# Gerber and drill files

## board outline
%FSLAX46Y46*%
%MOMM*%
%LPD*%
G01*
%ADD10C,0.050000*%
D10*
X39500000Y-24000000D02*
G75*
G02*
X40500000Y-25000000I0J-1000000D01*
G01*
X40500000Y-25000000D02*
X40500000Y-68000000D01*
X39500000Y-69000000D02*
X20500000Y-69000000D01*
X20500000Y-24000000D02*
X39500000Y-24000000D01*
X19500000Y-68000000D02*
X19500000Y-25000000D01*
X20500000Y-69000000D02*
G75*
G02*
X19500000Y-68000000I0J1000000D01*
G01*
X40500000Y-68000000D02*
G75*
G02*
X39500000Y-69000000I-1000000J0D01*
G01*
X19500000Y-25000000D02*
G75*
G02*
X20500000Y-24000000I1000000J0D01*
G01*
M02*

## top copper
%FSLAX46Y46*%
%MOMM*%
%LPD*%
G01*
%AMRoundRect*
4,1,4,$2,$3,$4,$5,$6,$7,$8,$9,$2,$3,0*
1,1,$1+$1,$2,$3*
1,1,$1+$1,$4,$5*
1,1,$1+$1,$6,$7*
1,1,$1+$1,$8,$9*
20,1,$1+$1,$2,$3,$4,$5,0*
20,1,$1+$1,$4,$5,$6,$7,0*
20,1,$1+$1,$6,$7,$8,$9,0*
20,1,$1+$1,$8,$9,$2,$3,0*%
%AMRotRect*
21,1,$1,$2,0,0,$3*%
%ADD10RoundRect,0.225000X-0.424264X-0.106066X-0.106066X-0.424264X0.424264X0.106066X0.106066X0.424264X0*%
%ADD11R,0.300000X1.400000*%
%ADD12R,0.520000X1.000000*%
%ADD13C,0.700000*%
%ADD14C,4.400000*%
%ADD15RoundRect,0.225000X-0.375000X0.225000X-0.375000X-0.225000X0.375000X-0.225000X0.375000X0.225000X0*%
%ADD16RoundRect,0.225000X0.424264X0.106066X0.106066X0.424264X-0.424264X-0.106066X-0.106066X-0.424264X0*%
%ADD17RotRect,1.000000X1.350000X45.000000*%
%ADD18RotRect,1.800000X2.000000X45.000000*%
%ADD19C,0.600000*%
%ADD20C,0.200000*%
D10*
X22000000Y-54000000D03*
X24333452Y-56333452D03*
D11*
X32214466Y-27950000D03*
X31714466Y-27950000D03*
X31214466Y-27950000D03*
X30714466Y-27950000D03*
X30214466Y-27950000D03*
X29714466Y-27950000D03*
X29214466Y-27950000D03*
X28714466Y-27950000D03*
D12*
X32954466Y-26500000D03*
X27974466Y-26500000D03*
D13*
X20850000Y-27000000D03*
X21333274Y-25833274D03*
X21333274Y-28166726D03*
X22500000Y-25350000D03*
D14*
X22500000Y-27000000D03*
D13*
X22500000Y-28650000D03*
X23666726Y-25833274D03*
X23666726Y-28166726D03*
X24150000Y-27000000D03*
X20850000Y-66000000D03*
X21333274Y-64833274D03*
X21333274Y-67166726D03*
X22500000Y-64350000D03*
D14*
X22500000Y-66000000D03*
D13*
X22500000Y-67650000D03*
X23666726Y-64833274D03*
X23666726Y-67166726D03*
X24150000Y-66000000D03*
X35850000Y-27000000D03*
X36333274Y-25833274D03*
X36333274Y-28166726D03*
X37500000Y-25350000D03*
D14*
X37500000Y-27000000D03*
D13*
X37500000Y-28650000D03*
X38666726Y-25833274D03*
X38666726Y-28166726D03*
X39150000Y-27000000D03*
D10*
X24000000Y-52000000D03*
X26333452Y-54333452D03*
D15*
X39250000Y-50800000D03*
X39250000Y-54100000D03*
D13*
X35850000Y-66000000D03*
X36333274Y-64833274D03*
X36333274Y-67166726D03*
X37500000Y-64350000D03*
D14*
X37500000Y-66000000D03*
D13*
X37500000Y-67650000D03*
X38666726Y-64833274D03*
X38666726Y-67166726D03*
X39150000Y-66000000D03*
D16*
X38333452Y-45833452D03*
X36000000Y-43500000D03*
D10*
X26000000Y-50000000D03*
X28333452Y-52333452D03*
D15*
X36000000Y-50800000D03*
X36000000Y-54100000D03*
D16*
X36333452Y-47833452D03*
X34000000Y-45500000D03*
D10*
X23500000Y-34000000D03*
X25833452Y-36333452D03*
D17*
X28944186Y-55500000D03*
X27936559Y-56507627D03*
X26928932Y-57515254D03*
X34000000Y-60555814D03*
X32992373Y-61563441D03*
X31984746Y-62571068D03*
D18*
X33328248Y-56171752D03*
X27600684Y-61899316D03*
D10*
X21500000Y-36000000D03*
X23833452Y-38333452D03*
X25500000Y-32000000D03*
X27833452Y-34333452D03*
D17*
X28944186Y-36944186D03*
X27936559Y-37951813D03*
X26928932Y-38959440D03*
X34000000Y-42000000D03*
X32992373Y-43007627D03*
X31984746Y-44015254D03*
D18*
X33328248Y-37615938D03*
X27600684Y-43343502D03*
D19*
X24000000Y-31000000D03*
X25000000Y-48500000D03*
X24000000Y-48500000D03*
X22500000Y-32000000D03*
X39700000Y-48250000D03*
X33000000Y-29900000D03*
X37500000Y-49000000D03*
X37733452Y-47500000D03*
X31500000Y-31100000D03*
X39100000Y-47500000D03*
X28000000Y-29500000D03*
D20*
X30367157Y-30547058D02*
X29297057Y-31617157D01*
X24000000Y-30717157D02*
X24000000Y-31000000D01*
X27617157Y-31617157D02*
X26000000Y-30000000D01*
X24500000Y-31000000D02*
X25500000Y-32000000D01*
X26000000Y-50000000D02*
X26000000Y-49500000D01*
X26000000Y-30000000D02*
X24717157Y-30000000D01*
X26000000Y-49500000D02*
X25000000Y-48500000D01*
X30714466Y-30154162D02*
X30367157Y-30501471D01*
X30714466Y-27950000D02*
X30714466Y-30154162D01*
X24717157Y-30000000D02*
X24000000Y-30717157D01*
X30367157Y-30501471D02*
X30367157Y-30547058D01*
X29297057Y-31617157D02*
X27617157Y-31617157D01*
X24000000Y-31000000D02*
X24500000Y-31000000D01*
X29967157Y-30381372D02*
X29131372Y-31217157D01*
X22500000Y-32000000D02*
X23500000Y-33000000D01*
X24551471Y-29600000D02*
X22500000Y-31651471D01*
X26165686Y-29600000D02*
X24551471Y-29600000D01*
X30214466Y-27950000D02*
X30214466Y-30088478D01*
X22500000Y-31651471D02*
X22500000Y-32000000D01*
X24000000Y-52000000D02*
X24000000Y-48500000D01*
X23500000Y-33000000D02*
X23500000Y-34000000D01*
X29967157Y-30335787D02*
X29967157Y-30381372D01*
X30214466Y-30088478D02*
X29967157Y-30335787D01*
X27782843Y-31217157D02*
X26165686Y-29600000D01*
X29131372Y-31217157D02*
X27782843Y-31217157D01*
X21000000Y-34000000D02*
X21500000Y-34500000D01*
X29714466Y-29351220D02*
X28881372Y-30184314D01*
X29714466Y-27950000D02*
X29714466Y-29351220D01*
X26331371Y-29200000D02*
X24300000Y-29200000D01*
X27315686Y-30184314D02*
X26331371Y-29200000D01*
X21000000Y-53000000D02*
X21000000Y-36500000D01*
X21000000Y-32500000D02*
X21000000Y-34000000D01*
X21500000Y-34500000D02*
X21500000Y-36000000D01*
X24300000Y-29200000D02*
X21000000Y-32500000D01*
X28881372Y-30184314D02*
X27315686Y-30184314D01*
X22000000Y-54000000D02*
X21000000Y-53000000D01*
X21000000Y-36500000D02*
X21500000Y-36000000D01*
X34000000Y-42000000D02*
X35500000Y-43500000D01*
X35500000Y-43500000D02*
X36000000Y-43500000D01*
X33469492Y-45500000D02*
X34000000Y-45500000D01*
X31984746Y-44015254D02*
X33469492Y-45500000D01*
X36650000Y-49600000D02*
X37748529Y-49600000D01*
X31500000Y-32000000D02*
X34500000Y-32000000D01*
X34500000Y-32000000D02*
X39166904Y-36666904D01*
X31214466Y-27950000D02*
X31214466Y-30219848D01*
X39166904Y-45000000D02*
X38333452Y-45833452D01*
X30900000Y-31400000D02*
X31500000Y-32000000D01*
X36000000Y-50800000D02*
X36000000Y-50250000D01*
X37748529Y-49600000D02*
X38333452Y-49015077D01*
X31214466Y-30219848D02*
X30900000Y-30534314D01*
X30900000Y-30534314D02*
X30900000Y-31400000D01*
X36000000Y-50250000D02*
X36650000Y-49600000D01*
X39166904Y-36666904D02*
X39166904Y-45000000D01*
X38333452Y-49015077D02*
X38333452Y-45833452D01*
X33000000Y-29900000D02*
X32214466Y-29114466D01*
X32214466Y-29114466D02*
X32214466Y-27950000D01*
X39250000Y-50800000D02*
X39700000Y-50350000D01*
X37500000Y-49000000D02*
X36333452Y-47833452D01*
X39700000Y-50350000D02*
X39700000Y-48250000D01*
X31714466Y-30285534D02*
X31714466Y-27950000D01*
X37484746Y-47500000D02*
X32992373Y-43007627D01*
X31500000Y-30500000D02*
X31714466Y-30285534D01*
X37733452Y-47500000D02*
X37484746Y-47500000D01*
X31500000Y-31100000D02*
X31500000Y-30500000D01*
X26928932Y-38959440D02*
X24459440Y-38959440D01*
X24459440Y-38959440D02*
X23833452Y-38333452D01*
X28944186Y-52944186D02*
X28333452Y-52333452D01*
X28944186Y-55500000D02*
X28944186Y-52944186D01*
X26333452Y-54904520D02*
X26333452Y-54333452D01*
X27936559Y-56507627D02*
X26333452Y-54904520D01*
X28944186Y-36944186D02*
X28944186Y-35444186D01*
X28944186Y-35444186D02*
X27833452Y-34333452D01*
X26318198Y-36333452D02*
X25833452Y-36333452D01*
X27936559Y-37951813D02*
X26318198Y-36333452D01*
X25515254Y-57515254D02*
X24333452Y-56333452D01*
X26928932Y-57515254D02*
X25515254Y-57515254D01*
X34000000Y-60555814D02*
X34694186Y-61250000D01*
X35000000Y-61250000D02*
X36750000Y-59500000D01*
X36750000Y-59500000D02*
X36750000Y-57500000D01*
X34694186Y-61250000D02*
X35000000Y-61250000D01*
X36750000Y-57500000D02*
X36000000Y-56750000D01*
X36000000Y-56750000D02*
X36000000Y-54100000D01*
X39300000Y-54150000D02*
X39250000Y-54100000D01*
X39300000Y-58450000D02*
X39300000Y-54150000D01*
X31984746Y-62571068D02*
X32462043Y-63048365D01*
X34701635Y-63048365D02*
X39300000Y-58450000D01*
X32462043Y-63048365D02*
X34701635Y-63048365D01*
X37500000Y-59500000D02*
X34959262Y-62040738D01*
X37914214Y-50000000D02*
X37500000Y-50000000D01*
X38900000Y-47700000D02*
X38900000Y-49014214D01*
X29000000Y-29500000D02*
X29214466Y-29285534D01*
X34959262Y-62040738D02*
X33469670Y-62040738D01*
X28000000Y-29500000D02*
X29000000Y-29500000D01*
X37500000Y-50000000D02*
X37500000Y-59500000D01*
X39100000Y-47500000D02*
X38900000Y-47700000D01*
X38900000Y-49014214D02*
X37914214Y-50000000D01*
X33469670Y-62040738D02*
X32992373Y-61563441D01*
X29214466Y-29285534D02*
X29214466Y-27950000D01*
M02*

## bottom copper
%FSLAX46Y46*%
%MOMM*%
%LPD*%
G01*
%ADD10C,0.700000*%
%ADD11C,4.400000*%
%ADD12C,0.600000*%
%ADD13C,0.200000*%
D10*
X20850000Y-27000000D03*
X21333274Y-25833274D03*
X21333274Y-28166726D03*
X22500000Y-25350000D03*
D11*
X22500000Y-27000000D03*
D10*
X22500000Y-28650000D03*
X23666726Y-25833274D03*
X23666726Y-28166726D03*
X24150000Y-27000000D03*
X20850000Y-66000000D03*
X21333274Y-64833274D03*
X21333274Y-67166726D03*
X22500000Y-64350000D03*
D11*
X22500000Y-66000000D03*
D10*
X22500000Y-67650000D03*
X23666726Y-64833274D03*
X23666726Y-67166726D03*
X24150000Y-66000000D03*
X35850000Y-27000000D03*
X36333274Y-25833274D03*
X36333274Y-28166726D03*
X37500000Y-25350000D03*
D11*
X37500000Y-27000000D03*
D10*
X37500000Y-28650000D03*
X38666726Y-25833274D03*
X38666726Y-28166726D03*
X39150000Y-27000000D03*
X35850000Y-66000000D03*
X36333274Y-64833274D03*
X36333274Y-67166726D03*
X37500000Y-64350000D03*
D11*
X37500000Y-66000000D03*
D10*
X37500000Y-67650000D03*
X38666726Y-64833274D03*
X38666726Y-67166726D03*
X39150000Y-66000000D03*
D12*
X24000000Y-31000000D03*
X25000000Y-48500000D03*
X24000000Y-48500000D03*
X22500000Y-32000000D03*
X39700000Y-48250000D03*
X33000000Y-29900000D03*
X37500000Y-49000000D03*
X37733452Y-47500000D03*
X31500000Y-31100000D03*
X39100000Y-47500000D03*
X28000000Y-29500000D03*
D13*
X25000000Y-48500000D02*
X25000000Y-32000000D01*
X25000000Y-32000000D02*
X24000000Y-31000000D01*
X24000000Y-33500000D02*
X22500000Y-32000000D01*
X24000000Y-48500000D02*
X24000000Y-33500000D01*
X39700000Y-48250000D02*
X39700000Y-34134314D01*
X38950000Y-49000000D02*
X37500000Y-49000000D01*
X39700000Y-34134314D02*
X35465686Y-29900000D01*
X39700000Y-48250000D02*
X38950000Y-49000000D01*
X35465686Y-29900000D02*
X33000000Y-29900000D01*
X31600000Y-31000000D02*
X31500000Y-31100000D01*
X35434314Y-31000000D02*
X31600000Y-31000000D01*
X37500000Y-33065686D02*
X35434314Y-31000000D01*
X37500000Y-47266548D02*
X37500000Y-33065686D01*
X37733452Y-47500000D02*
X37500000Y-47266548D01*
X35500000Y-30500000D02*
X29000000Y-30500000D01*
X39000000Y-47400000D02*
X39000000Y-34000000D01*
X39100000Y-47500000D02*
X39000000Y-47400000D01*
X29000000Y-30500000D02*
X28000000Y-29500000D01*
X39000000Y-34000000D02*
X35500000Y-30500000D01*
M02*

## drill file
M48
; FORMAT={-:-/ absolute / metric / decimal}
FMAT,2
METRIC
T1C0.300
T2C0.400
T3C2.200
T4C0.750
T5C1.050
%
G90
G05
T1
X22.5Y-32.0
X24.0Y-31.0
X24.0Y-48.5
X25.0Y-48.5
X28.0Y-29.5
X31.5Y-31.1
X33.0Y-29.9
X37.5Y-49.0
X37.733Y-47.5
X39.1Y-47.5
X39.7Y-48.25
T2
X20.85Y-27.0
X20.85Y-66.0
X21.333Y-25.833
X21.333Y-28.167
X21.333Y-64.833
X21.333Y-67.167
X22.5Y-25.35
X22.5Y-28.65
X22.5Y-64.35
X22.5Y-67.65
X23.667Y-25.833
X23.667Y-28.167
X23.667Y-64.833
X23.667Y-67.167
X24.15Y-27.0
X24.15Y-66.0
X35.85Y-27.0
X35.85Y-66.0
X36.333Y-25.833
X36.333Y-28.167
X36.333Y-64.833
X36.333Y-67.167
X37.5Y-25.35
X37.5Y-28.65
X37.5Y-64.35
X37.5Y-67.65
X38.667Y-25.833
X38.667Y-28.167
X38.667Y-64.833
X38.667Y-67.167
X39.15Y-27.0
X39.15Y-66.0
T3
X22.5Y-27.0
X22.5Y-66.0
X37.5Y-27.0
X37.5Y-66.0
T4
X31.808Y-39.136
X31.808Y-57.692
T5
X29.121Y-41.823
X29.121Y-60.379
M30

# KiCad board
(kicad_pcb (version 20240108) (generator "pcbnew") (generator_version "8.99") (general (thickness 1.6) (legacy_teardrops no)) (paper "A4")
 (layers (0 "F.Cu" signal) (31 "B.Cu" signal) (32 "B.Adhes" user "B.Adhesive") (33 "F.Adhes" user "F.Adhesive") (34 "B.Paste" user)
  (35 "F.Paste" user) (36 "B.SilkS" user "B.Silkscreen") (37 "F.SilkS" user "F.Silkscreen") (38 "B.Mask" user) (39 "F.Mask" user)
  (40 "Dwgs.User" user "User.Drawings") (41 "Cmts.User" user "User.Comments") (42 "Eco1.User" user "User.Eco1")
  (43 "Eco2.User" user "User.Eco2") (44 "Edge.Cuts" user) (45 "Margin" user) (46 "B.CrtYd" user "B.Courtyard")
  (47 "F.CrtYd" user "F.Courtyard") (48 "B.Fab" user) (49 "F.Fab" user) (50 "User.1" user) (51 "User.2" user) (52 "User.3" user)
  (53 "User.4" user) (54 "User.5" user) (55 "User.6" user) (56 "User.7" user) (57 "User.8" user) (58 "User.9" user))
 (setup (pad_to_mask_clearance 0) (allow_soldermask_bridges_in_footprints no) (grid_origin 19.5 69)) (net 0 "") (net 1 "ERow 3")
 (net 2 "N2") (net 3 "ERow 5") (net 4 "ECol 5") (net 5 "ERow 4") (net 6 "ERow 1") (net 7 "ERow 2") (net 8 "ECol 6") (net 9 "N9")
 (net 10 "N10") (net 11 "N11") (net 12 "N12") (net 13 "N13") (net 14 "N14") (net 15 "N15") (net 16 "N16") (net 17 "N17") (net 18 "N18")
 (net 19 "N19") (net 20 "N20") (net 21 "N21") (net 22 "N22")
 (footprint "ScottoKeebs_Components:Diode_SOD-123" (layer "F.Cu") (at 23.166726 55.166726 -45)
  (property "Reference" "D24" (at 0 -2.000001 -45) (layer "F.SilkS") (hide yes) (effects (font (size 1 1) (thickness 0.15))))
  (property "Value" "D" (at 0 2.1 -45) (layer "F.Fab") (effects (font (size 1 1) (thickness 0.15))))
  (pad "1" smd roundrect (at -1.65 0 315) (size 0.9 1.2) (layers "F.Cu" "F.Paste" "F.Mask") (roundrect_rratio 0.25) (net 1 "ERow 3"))
  (pad "2" smd roundrect (at 1.65 0 315) (size 0.9 1.2) (layers "F.Cu" "F.Paste" "F.Mask") (roundrect_rratio 0.25) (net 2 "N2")))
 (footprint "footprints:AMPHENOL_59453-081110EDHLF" (layer "F.Cu") (at 30.464466 26.1 180)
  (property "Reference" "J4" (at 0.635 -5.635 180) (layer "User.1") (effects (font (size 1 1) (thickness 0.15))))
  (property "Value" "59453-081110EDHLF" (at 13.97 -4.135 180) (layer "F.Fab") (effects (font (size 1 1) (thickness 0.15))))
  (pad "1" smd rect (at -1.75 -1.85 180) (size 0.3 1.4) (layers "F.Cu" "F.Paste") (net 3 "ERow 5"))
  (pad "2" smd rect (at -1.25 -1.85 180) (size 0.3 1.4) (layers "F.Cu" "F.Paste") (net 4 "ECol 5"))
  (pad "3" smd rect (at -0.75 -1.85 180) (size 0.3 1.4) (layers "F.Cu" "F.Paste") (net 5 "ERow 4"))
  (pad "4" smd rect (at -0.25 -1.85 180) (size 0.3 1.4) (layers "F.Cu" "F.Paste") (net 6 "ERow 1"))
  (pad "5" smd rect (at 0.25 -1.85 180) (size 0.3 1.4) (layers "F.Cu" "F.Paste") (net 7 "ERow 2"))
  (pad "6" smd rect (at 0.75 -1.85 180) (size 0.3 1.4) (layers "F.Cu" "F.Paste") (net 1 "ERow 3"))
  (pad "7" smd rect (at 1.25 -1.85 180) (size 0.3 1.4) (layers "F.Cu" "F.Paste") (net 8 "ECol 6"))
  (pad "8" smd rect (at 1.75 -1.85 180) (size 0.3 1.4) (layers "F.Cu" "F.Paste") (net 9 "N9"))
  (pad "SH1" smd rect (at -2.49 -0.4 180) (size 0.52 1) (layers "F.Cu" "F.Paste" "F.Mask") (solder_mask_margin 0.102))
  (pad "SH2" smd rect (at 2.49 -0.4 180) (size 0.52 1) (layers "F.Cu" "F.Paste" "F.Mask") (solder_mask_margin 0.102)))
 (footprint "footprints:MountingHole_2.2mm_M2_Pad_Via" (layer "F.Cu") (at 22.5 27)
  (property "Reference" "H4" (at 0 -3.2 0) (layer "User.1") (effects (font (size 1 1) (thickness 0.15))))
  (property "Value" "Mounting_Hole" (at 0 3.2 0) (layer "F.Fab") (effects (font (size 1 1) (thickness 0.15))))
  (pad "1" thru_hole circle (at -1.65 0) (size 0.7 0.7) (drill 0.4) (layers "*.Cu" "*.Mask") (remove_unused_layers no) (zone_connect 2))
  (pad "1" thru_hole circle (at -1.166726 -1.166726) (size 0.7 0.7) (drill 0.4) (layers "*.Cu" "*.Mask") (remove_unused_layers no)
   (zone_connect 2))
  (pad "1" thru_hole circle (at -1.166726 1.166726) (size 0.7 0.7) (drill 0.4) (layers "*.Cu" "*.Mask") (remove_unused_layers no)
   (zone_connect 2))
  (pad "1" thru_hole circle (at 0 -1.65) (size 0.7 0.7) (drill 0.4) (layers "*.Cu" "*.Mask") (remove_unused_layers no) (zone_connect 2))
  (pad "1" thru_hole circle (at 0 0) (size 4.4 4.4) (drill 2.2) (layers "*.Cu" "*.Mask") (remove_unused_layers no))
  (pad "1" thru_hole circle (at 0 1.65) (size 0.7 0.7) (drill 0.4) (layers "*.Cu" "*.Mask") (remove_unused_layers no) (zone_connect 2))
  (pad "1" thru_hole circle (at 1.166726 -1.166726) (size 0.7 0.7) (drill 0.4) (layers "*.Cu" "*.Mask") (remove_unused_layers no)
   (zone_connect 2))
  (pad "1" thru_hole circle (at 1.166726 1.166726) (size 0.7 0.7) (drill 0.4) (layers "*.Cu" "*.Mask") (remove_unused_layers no)
   (zone_connect 2))
  (pad "1" thru_hole circle (at 1.65 0) (size 0.7 0.7) (drill 0.4) (layers "*.Cu" "*.Mask") (remove_unused_layers no) (zone_connect 2)))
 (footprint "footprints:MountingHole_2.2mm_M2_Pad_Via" (layer "F.Cu") (at 22.5 66)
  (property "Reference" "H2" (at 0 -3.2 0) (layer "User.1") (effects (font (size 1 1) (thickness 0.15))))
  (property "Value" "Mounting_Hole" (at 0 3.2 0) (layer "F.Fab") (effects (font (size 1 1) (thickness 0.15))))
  (pad "1" thru_hole circle (at -1.65 0) (size 0.7 0.7) (drill 0.4) (layers "*.Cu" "*.Mask") (remove_unused_layers no) (zone_connect 2))
  (pad "1" thru_hole circle (at -1.166726 -1.166726) (size 0.7 0.7) (drill 0.4) (layers "*.Cu" "*.Mask") (remove_unused_layers no)
   (zone_connect 2))
  (pad "1" thru_hole circle (at -1.166726 1.166726) (size 0.7 0.7) (drill 0.4) (layers "*.Cu" "*.Mask") (remove_unused_layers no)
   (zone_connect 2))
  (pad "1" thru_hole circle (at 0 -1.65) (size 0.7 0.7) (drill 0.4) (layers "*.Cu" "*.Mask") (remove_unused_layers no) (zone_connect 2))
  (pad "1" thru_hole circle (at 0 0) (size 4.4 4.4) (drill 2.2) (layers "*.Cu" "*.Mask") (remove_unused_layers no))
  (pad "1" thru_hole circle (at 0 1.65) (size 0.7 0.7) (drill 0.4) (layers "*.Cu" "*.Mask") (remove_unused_layers no) (zone_connect 2))
  (pad "1" thru_hole circle (at 1.166726 -1.166726) (size 0.7 0.7) (drill 0.4) (layers "*.Cu" "*.Mask") (remove_unused_layers no)
   (zone_connect 2))
  (pad "1" thru_hole circle (at 1.166726 1.166726) (size 0.7 0.7) (drill 0.4) (layers "*.Cu" "*.Mask") (remove_unused_layers no)
   (zone_connect 2))
  (pad "1" thru_hole circle (at 1.65 0) (size 0.7 0.7) (drill 0.4) (layers "*.Cu" "*.Mask") (remove_unused_layers no) (zone_connect 2)))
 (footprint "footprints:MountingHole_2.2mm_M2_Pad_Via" (layer "F.Cu") (at 37.5 27)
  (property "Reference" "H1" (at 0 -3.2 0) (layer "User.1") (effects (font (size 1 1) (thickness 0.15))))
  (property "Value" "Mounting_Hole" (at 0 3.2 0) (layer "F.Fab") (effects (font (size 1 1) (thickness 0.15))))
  (pad "1" thru_hole circle (at -1.65 0) (size 0.7 0.7) (drill 0.4) (layers "*.Cu" "*.Mask") (remove_unused_layers no) (zone_connect 2))
  (pad "1" thru_hole circle (at -1.166726 -1.166726) (size 0.7 0.7) (drill 0.4) (layers "*.Cu" "*.Mask") (remove_unused_layers no)
   (zone_connect 2))
  (pad "1" thru_hole circle (at -1.166726 1.166726) (size 0.7 0.7) (drill 0.4) (layers "*.Cu" "*.Mask") (remove_unused_layers no)
   (zone_connect 2))
  (pad "1" thru_hole circle (at 0 -1.65) (size 0.7 0.7) (drill 0.4) (layers "*.Cu" "*.Mask") (remove_unused_layers no) (zone_connect 2))
  (pad "1" thru_hole circle (at 0 0) (size 4.4 4.4) (drill 2.2) (layers "*.Cu" "*.Mask") (remove_unused_layers no))
  (pad "1" thru_hole circle (at 0 1.65) (size 0.7 0.7) (drill 0.4) (layers "*.Cu" "*.Mask") (remove_unused_layers no) (zone_connect 2))
  (pad "1" thru_hole circle (at 1.166726 -1.166726) (size 0.7 0.7) (drill 0.4) (layers "*.Cu" "*.Mask") (remove_unused_layers no)
   (zone_connect 2))
  (pad "1" thru_hole circle (at 1.166726 1.166726) (size 0.7 0.7) (drill 0.4) (layers "*.Cu" "*.Mask") (remove_unused_layers no)
   (zone_connect 2))
  (pad "1" thru_hole circle (at 1.65 0) (size 0.7 0.7) (drill 0.4) (layers "*.Cu" "*.Mask") (remove_unused_layers no) (zone_connect 2)))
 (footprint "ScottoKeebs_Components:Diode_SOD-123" (layer "F.Cu") (at 25.166726 53.166726 -45)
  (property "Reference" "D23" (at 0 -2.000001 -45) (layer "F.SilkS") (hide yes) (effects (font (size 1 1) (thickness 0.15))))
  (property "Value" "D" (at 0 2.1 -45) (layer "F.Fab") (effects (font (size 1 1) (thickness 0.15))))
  (pad "1" smd roundrect (at -1.65 0 315) (size 0.9 1.2) (layers "F.Cu" "F.Paste" "F.Mask") (roundrect_rratio 0.25) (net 7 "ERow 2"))
  (pad "2" smd roundrect (at 1.65 0 315) (size 0.9 1.2) (layers "F.Cu" "F.Paste" "F.Mask") (roundrect_rratio 0.25) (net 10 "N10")))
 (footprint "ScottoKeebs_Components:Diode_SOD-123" (layer "F.Cu") (at 39.25 52.45 -90)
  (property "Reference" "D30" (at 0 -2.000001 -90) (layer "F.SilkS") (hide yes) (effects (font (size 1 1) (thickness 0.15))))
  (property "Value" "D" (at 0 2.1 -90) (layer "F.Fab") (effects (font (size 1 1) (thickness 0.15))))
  (pad "1" smd roundrect (at -1.65 0 270) (size 0.9 1.2) (layers "F.Cu" "F.Paste" "F.Mask") (roundrect_rratio 0.25) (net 3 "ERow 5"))
  (pad "2" smd roundrect (at 1.65 0 270) (size 0.9 1.2) (layers "F.Cu" "F.Paste" "F.Mask") (roundrect_rratio 0.25) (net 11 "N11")))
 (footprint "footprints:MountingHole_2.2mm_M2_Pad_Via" (layer "F.Cu") (at 37.5 66)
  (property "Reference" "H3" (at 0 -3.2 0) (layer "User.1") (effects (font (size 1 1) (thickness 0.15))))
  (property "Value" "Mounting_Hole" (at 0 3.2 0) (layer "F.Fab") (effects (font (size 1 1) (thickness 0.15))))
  (pad "1" thru_hole circle (at -1.65 0) (size 0.7 0.7) (drill 0.4) (layers "*.Cu" "*.Mask") (remove_unused_layers no) (zone_connect 2))
  (pad "1" thru_hole circle (at -1.166726 -1.166726) (size 0.7 0.7) (drill 0.4) (layers "*.Cu" "*.Mask") (remove_unused_layers no)
   (zone_connect 2))
  (pad "1" thru_hole circle (at -1.166726 1.166726) (size 0.7 0.7) (drill 0.4) (layers "*.Cu" "*.Mask") (remove_unused_layers no)
   (zone_connect 2))
  (pad "1" thru_hole circle (at 0 -1.65) (size 0.7 0.7) (drill 0.4) (layers "*.Cu" "*.Mask") (remove_unused_layers no) (zone_connect 2))
  (pad "1" thru_hole circle (at 0 0) (size 4.4 4.4) (drill 2.2) (layers "*.Cu" "*.Mask") (remove_unused_layers no))
  (pad "1" thru_hole circle (at 0 1.65) (size 0.7 0.7) (drill 0.4) (layers "*.Cu" "*.Mask") (remove_unused_layers no) (zone_connect 2))
  (pad "1" thru_hole circle (at 1.166726 -1.166726) (size 0.7 0.7) (drill 0.4) (layers "*.Cu" "*.Mask") (remove_unused_layers no)
   (zone_connect 2))
  (pad "1" thru_hole circle (at 1.166726 1.166726) (size 0.7 0.7) (drill 0.4) (layers "*.Cu" "*.Mask") (remove_unused_layers no)
   (zone_connect 2))
  (pad "1" thru_hole circle (at 1.65 0) (size 0.7 0.7) (drill 0.4) (layers "*.Cu" "*.Mask") (remove_unused_layers no) (zone_connect 2)))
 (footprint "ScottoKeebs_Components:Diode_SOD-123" (layer "F.Cu") (at 37.166726 44.666726 135)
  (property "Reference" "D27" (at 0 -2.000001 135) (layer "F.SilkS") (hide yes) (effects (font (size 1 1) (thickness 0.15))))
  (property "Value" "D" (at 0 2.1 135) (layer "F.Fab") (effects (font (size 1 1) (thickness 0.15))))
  (pad "1" smd roundrect (at -1.65 0 135) (size 0.9 1.2) (layers "F.Cu" "F.Paste" "F.Mask") (roundrect_rratio 0.25) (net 5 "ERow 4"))
  (pad "2" smd roundrect (at 1.65 0 135) (size 0.9 1.2) (layers "F.Cu" "F.Paste" "F.Mask") (roundrect_rratio 0.25) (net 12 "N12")))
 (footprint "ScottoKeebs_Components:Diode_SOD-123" (layer "F.Cu") (at 27.166726 51.166726 -45)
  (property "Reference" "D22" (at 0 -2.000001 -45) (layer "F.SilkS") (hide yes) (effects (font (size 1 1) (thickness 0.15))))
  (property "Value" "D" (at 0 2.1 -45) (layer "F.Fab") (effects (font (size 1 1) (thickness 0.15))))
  (pad "1" smd roundrect (at -1.65 0 315) (size 0.9 1.2) (layers "F.Cu" "F.Paste" "F.Mask") (roundrect_rratio 0.25) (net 6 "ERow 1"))
  (pad "2" smd roundrect (at 1.65 0 315) (size 0.9 1.2) (layers "F.Cu" "F.Paste" "F.Mask") (roundrect_rratio 0.25) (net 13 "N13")))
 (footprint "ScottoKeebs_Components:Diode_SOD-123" (layer "F.Cu") (at 36 52.45 -90)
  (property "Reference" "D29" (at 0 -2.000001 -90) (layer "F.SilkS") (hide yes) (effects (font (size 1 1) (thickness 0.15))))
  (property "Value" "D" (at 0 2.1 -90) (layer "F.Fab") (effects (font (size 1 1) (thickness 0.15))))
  (pad "1" smd roundrect (at -1.65 0 270) (size 0.9 1.2) (layers "F.Cu" "F.Paste" "F.Mask") (roundrect_rratio 0.25) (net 5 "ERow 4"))
  (pad "2" smd roundrect (at 1.65 0 270) (size 0.9 1.2) (layers "F.Cu" "F.Paste" "F.Mask") (roundrect_rratio 0.25) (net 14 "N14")))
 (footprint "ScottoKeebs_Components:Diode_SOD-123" (layer "F.Cu") (at 35.166726 46.666726 135)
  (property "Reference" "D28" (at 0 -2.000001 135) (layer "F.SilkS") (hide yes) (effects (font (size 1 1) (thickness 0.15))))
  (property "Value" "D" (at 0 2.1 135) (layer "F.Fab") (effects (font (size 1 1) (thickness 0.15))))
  (pad "1" smd roundrect (at -1.65 0 135) (size 0.9 1.2) (layers "F.Cu" "F.Paste" "F.Mask") (roundrect_rratio 0.25) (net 3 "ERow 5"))
  (pad "2" smd roundrect (at 1.65 0 135) (size 0.9 1.2) (layers "F.Cu" "F.Paste" "F.Mask") (roundrect_rratio 0.25) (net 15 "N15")))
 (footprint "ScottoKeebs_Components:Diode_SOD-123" (layer "F.Cu") (at 24.666726 35.166726 -45)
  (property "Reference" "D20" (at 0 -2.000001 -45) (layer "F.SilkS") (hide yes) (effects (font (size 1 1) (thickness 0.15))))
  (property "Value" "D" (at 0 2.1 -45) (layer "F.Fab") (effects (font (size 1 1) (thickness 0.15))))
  (pad "1" smd roundrect (at -1.65 0 315) (size 0.9 1.2) (layers "F.Cu" "F.Paste" "F.Mask") (roundrect_rratio 0.25) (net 7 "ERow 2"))
  (pad "2" smd roundrect (at 1.65 0 315) (size 0.9 1.2) (layers "F.Cu" "F.Paste" "F.Mask") (roundrect_rratio 0.25) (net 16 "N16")))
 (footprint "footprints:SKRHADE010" (layer "F.Cu") (at 30.464466 59.035534 -45)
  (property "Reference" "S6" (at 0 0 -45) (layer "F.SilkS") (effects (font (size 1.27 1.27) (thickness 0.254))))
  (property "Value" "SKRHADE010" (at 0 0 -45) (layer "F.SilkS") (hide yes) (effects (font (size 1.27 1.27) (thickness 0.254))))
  (pad "" np_thru_hole circle (at 0 -1.9 315) (size 0.75 0.75) (drill 0.75) (layers "*.Cu" "*.Mask"))
  (pad "" np_thru_hole circle (at 0 1.9 315) (size 1.05 1.05) (drill 1.05) (layers "*.Cu" "*.Mask"))
  (pad "1" smd rect (at -3.575 -1.425 45) (size 1 1.35) (layers "F.Cu" "F.Paste" "F.Mask") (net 13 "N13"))
  (pad "2" smd rect (at -3.575 0 45) (size 1 1.35) (layers "F.Cu" "F.Paste" "F.Mask") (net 10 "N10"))
  (pad "3" smd rect (at -3.575 1.425 45) (size 1 1.35) (layers "F.Cu" "F.Paste" "F.Mask") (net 2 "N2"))
  (pad "4" smd rect (at 3.575 -1.425 45) (size 1 1.35) (layers "F.Cu" "F.Paste" "F.Mask") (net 14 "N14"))
  (pad "5" smd rect (at 3.575 0 45) (size 1 1.35) (layers "F.Cu" "F.Paste" "F.Mask") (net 8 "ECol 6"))
  (pad "6" smd rect (at 3.575 1.425 45) (size 1 1.35) (layers "F.Cu" "F.Paste" "F.Mask") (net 11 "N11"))
  (pad "MP1" smd rect (at 0 -4.049999 45) (size 1.8 2) (layers "F.Cu" "F.Paste" "F.Mask") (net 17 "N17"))
  (pad "MP2" smd rect (at 0 4.049999 45) (size 1.8 2) (layers "F.Cu" "F.Paste" "F.Mask") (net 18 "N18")))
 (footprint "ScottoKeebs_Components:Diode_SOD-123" (layer "F.Cu") (at 22.666726 37.166726 -45)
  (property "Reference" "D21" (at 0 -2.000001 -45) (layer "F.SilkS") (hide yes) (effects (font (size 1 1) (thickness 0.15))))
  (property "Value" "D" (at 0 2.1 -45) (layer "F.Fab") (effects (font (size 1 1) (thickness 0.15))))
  (pad "1" smd roundrect (at -1.65 0 315) (size 0.9 1.2) (layers "F.Cu" "F.Paste" "F.Mask") (roundrect_rratio 0.25) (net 1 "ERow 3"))
  (pad "2" smd roundrect (at 1.65 0 315) (size 0.9 1.2) (layers "F.Cu" "F.Paste" "F.Mask") (roundrect_rratio 0.25) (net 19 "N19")))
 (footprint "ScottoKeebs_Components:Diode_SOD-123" (layer "F.Cu") (at 26.666726 33.166726 -45)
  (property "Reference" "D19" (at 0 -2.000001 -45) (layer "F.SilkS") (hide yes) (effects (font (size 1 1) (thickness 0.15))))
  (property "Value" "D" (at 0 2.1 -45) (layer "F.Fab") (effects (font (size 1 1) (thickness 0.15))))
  (pad "1" smd roundrect (at -1.65 0 315) (size 0.9 1.2) (layers "F.Cu" "F.Paste" "F.Mask") (roundrect_rratio 0.25) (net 6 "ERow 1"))
  (pad "2" smd roundrect (at 1.65 0 315) (size 0.9 1.2) (layers "F.Cu" "F.Paste" "F.Mask") (roundrect_rratio 0.25) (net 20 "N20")))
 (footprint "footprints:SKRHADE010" (layer "F.Cu") (at 30.464466 40.47972 -45)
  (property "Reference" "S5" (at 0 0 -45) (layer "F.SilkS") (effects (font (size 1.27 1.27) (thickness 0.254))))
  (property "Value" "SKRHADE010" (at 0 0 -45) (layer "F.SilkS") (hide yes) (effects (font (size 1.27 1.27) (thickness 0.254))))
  (pad "" np_thru_hole circle (at 0 -1.9 315) (size 0.75 0.75) (drill 0.75) (layers "*.Cu" "*.Mask"))
  (pad "" np_thru_hole circle (at 0 1.9 315) (size 1.05 1.05) (drill 1.05) (layers "*.Cu" "*.Mask"))
  (pad "1" smd rect (at -3.575 -1.425 45) (size 1 1.35) (layers "F.Cu" "F.Paste" "F.Mask") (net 20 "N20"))
  (pad "2" smd rect (at -3.575 0 45) (size 1 1.35) (layers "F.Cu" "F.Paste" "F.Mask") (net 16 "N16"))
  (pad "3" smd rect (at -3.575 1.425 45) (size 1 1.35) (layers "F.Cu" "F.Paste" "F.Mask") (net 19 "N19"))
  (pad "4" smd rect (at 3.575 -1.425 45) (size 1 1.35) (layers "F.Cu" "F.Paste" "F.Mask") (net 12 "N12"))
  (pad "5" smd rect (at 3.575 0 45) (size 1 1.35) (layers "F.Cu" "F.Paste" "F.Mask") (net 4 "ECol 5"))
  (pad "6" smd rect (at 3.575 1.425 45) (size 1 1.35) (layers "F.Cu" "F.Paste" "F.Mask") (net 15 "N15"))
  (pad "MP1" smd rect (at 0 -4.049999 45) (size 1.8 2) (layers "F.Cu" "F.Paste" "F.Mask") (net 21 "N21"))
  (pad "MP2" smd rect (at 0 4.049999 45) (size 1.8 2) (layers "F.Cu" "F.Paste" "F.Mask") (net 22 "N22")))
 (gr_arc (start 39.5 24) (mid 40.207107 24.292893) (end 40.5 25) (stroke (width 0.05) (type default)) (layer "Edge.Cuts"))
 (gr_line (start 40.5 25) (end 40.5 68) (stroke (width 0.05) (type default)) (layer "Edge.Cuts"))
 (gr_line (start 39.5 69) (end 20.5 69) (stroke (width 0.05) (type default)) (layer "Edge.Cuts"))
 (gr_line (start 20.5 24) (end 39.5 24) (stroke (width 0.05) (type default)) (layer "Edge.Cuts"))
 (gr_line (start 19.5 68) (end 19.5 25) (stroke (width 0.05) (type default)) (layer "Edge.Cuts"))
 (gr_arc (start 20.5 69) (mid 19.792893 68.707107) (end 19.5 68) (stroke (width 0.05) (type default)) (layer "Edge.Cuts"))
 (gr_arc (start 40.5 68) (mid 40.207107 68.707107) (end 39.5 69) (stroke (width 0.05) (type default)) (layer "Edge.Cuts"))
 (gr_arc (start 19.5 25) (mid 19.792893 24.292893) (end 20.5 24) (stroke (width 0.05) (type default)) (layer "Edge.Cuts"))
 (segment (start 30.367157 30.547058) (end 29.297057 31.617157) (width 0.2) (layer "F.Cu") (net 6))
 (segment (start 24 30.717157) (end 24 31) (width 0.2) (layer "F.Cu") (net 6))
 (segment (start 27.617157 31.617157) (end 26 30) (width 0.2) (layer "F.Cu") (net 6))
 (segment (start 24.5 31) (end 25.5 32) (width 0.2) (layer "F.Cu") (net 6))
 (segment (start 26 50) (end 26 49.5) (width 0.2) (layer "F.Cu") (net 6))
 (segment (start 26 30) (end 24.717157 30) (width 0.2) (layer "F.Cu") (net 6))
 (segment (start 26 49.5) (end 25 48.5) (width 0.2) (layer "F.Cu") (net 6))
 (segment (start 30.714466 30.154162) (end 30.367157 30.501471) (width 0.2) (layer "F.Cu") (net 6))
 (segment (start 30.714466 27.95) (end 30.714466 30.154162) (width 0.2) (layer "F.Cu") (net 6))
 (segment (start 24.717157 30) (end 24 30.717157) (width 0.2) (layer "F.Cu") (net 6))
 (segment (start 30.367157 30.501471) (end 30.367157 30.547058) (width 0.2) (layer "F.Cu") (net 6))
 (segment (start 29.297057 31.617157) (end 27.617157 31.617157) (width 0.2) (layer "F.Cu") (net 6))
 (segment (start 24 31) (end 24.5 31) (width 0.2) (layer "F.Cu") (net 6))
 (via (at 24 31) (size 0.6) (drill 0.3) (layers "F.Cu" "B.Cu") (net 6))
 (via (at 25 48.5) (size 0.6) (drill 0.3) (layers "F.Cu" "B.Cu") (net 6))
 (segment (start 25 48.5) (end 25 32) (width 0.2) (layer "B.Cu") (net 6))
 (segment (start 25 32) (end 24 31) (width 0.2) (layer "B.Cu") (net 6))
 (segment (start 29.967157 30.381372) (end 29.131372 31.217157) (width 0.2) (layer "F.Cu") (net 7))
 (segment (start 22.5 32) (end 23.5 33) (width 0.2) (layer "F.Cu") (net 7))
 (segment (start 24.551471 29.6) (end 22.5 31.651471) (width 0.2) (layer "F.Cu") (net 7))
 (segment (start 26.165686 29.6) (end 24.551471 29.6) (width 0.2) (layer "F.Cu") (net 7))
 (segment (start 30.214466 27.95) (end 30.214466 30.088478) (width 0.2) (layer "F.Cu") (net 7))
 (segment (start 22.5 31.651471) (end 22.5 32) (width 0.2) (layer "F.Cu") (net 7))
 (segment (start 24 52) (end 24 48.5) (width 0.2) (layer "F.Cu") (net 7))
 (segment (start 23.5 33) (end 23.5 34) (width 0.2) (layer "F.Cu") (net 7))
 (segment (start 29.967157 30.335787) (end 29.967157 30.381372) (width 0.2) (layer "F.Cu") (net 7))
 (segment (start 30.214466 30.088478) (end 29.967157 30.335787) (width 0.2) (layer "F.Cu") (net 7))
 (segment (start 27.782843 31.217157) (end 26.165686 29.6) (width 0.2) (layer "F.Cu") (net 7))
 (segment (start 29.131372 31.217157) (end 27.782843 31.217157) (width 0.2) (layer "F.Cu") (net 7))
 (via (at 24 48.5) (size 0.6) (drill 0.3) (layers "F.Cu" "B.Cu") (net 7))
 (via (at 22.5 32) (size 0.6) (drill 0.3) (layers "F.Cu" "B.Cu") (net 7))
 (segment (start 24 33.5) (end 22.5 32) (width 0.2) (layer "B.Cu") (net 7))
 (segment (start 24 48.5) (end 24 33.5) (width 0.2) (layer "B.Cu") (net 7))
 (segment (start 21 34) (end 21.5 34.5) (width 0.2) (layer "F.Cu") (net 1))
 (segment (start 29.714466 29.35122) (end 28.881372 30.184314) (width 0.2) (layer "F.Cu") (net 1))
 (segment (start 29.714466 27.95) (end 29.714466 29.35122) (width 0.2) (layer "F.Cu") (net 1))
 (segment (start 26.331371 29.2) (end 24.3 29.2) (width 0.2) (layer "F.Cu") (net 1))
 (segment (start 27.315686 30.184314) (end 26.331371 29.2) (width 0.2) (layer "F.Cu") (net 1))
 (segment (start 21 53) (end 21 36.5) (width 0.2) (layer "F.Cu") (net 1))
 (segment (start 21 32.5) (end 21 34) (width 0.2) (layer "F.Cu") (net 1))
 (segment (start 21.5 34.5) (end 21.5 36) (width 0.2) (layer "F.Cu") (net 1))
 (segment (start 24.3 29.2) (end 21 32.5) (width 0.2) (layer "F.Cu") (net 1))
 (segment (start 28.881372 30.184314) (end 27.315686 30.184314) (width 0.2) (layer "F.Cu") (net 1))
 (segment (start 22 54) (end 21 53) (width 0.2) (layer "F.Cu") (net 1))
 (segment (start 21 36.5) (end 21.5 36) (width 0.2) (layer "F.Cu") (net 1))
 (segment (start 34 42) (end 35.5 43.5) (width 0.2) (layer "F.Cu") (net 12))
 (segment (start 35.5 43.5) (end 36 43.5) (width 0.2) (layer "F.Cu") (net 12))
 (segment (start 33.469492 45.5) (end 34 45.5) (width 0.2) (layer "F.Cu") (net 15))
 (segment (start 31.984746 44.015254) (end 33.469492 45.5) (width 0.2) (layer "F.Cu") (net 15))
 (segment (start 36.65 49.6) (end 37.748529 49.6) (width 0.2) (layer "F.Cu") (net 5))
 (segment (start 31.5 32) (end 34.5 32) (width 0.2) (layer "F.Cu") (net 5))
 (segment (start 34.5 32) (end 39.166904 36.666904) (width 0.2) (layer "F.Cu") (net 5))
 (segment (start 31.214466 27.95) (end 31.214466 30.219848) (width 0.2) (layer "F.Cu") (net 5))
 (segment (start 39.166904 45) (end 38.333452 45.833452) (width 0.2) (layer "F.Cu") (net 5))
 (segment (start 30.9 31.4) (end 31.5 32) (width 0.2) (layer "F.Cu") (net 5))
 (segment (start 36 50.8) (end 36 50.25) (width 0.2) (layer "F.Cu") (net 5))
 (segment (start 37.748529 49.6) (end 38.333452 49.015077) (width 0.2) (layer "F.Cu") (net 5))
 (segment (start 31.214466 30.219848) (end 30.9 30.534314) (width 0.2) (layer "F.Cu") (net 5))
 (segment (start 30.9 30.534314) (end 30.9 31.4) (width 0.2) (layer "F.Cu") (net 5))
 (segment (start 36 50.25) (end 36.65 49.6) (width 0.2) (layer "F.Cu") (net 5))
 (segment (start 39.166904 36.666904) (end 39.166904 45) (width 0.2) (layer "F.Cu") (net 5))
 (segment (start 38.333452 49.015077) (end 38.333452 45.833452) (width 0.2) (layer "F.Cu") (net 5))
 (segment (start 33 29.9) (end 32.214466 29.114466) (width 0.2) (layer "F.Cu") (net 3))
 (segment (start 32.214466 29.114466) (end 32.214466 27.95) (width 0.2) (layer "F.Cu") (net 3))
 (segment (start 39.25 50.8) (end 39.7 50.35) (width 0.2) (layer "F.Cu") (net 3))
 (segment (start 37.5 49) (end 36.333452 47.833452) (width 0.2) (layer "F.Cu") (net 3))
 (segment (start 39.7 50.35) (end 39.7 48.25) (width 0.2) (layer "F.Cu") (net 3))
 (via (at 39.7 48.25) (size 0.6) (drill 0.3) (layers "F.Cu" "B.Cu") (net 3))
 (via (at 33 29.9) (size 0.6) (drill 0.3) (layers "F.Cu" "B.Cu") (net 3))
 (via (at 37.5 49) (size 0.6) (drill 0.3) (layers "F.Cu" "B.Cu") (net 3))
 (segment (start 39.7 48.25) (end 39.7 34.134314) (width 0.2) (layer "B.Cu") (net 3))
 (segment (start 38.95 49) (end 37.5 49) (width 0.2) (layer "B.Cu") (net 3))
 (segment (start 39.7 34.134314) (end 35.465686 29.9) (width 0.2) (layer "B.Cu") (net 3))
 (segment (start 39.7 48.25) (end 38.95 49) (width 0.2) (layer "B.Cu") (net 3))
 (segment (start 35.465686 29.9) (end 33 29.9) (width 0.2) (layer "B.Cu") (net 3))
 (segment (start 31.714466 30.285534) (end 31.714466 27.95) (width 0.2) (layer "F.Cu") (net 4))
 (segment (start 37.484746 47.5) (end 32.992373 43.007627) (width 0.2) (layer "F.Cu") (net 4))
 (segment (start 31.5 30.5) (end 31.714466 30.285534) (width 0.2) (layer "F.Cu") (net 4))
 (segment (start 37.733452 47.5) (end 37.484746 47.5) (width 0.2) (layer "F.Cu") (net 4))
 (segment (start 31.5 31.1) (end 31.5 30.5) (width 0.2) (layer "F.Cu") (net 4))
 (via (at 37.733452 47.5) (size 0.6) (drill 0.3) (layers "F.Cu" "B.Cu") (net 4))
 (via (at 31.5 31.1) (size 0.6) (drill 0.3) (layers "F.Cu" "B.Cu") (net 4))
 (segment (start 31.6 31) (end 31.5 31.1) (width 0.2) (layer "B.Cu") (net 4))
 (segment (start 35.434314 31) (end 31.6 31) (width 0.2) (layer "B.Cu") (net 4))
 (segment (start 37.5 33.065686) (end 35.434314 31) (width 0.2) (layer "B.Cu") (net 4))
 (segment (start 37.5 47.266548) (end 37.5 33.065686) (width 0.2) (layer "B.Cu") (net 4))
 (segment (start 37.733452 47.5) (end 37.5 47.266548) (width 0.2) (layer "B.Cu") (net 4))
 (segment (start 26.928932 38.95944) (end 24.45944 38.95944) (width 0.2) (layer "F.Cu") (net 19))
 (segment (start 24.45944 38.95944) (end 23.833452 38.333452) (width 0.2) (layer "F.Cu") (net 19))
 (segment (start 28.944186 52.944186) (end 28.333452 52.333452) (width 0.2) (layer "F.Cu") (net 13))
 (segment (start 28.944186 55.5) (end 28.944186 52.944186) (width 0.2) (layer "F.Cu") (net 13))
 (segment (start 26.333452 54.90452) (end 26.333452 54.333452) (width 0.2) (layer "F.Cu") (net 10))
 (segment (start 27.936559 56.507627) (end 26.333452 54.90452) (width 0.2) (layer "F.Cu") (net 10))
 (segment (start 28.944186 36.944186) (end 28.944186 35.444186) (width 0.2) (layer "F.Cu") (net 20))
 (segment (start 28.944186 35.444186) (end 27.833452 34.333452) (width 0.2) (layer "F.Cu") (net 20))
 (segment (start 26.318198 36.333452) (end 25.833452 36.333452) (width 0.2) (layer "F.Cu") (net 16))
 (segment (start 27.936559 37.951813) (end 26.318198 36.333452) (width 0.2) (layer "F.Cu") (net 16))
 (segment (start 25.515254 57.515254) (end 24.333452 56.333452) (width 0.2) (layer "F.Cu") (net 2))
 (segment (start 26.928932 57.515254) (end 25.515254 57.515254) (width 0.2) (layer "F.Cu") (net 2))
 (segment (start 34 60.555814) (end 34.694186 61.25) (width 0.2) (layer "F.Cu") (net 14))
 (segment (start 35 61.25) (end 36.75 59.5) (width 0.2) (layer "F.Cu") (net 14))
 (segment (start 36.75 59.5) (end 36.75 57.5) (width 0.2) (layer "F.Cu") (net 14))
 (segment (start 34.694186 61.25) (end 35 61.25) (width 0.2) (layer "F.Cu") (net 14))
 (segment (start 36.75 57.5) (end 36 56.75) (width 0.2) (layer "F.Cu") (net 14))
 (segment (start 36 56.75) (end 36 54.1) (width 0.2) (layer "F.Cu") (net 14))
 (segment (start 39.3 54.15) (end 39.25 54.1) (width 0.2) (layer "F.Cu") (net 11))
 (segment (start 39.3 58.45) (end 39.3 54.15) (width 0.2) (layer "F.Cu") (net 11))
 (segment (start 31.984746 62.571068) (end 32.462043 63.048365) (width 0.2) (layer "F.Cu") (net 11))
 (segment (start 34.701635 63.048365) (end 39.3 58.45) (width 0.2) (layer "F.Cu") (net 11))
 (segment (start 32.462043 63.048365) (end 34.701635 63.048365) (width 0.2) (layer "F.Cu") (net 11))
 (segment (start 37.5 59.5) (end 34.959262 62.040738) (width 0.2) (layer "F.Cu") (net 8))
 (segment (start 37.914214 50) (end 37.5 50) (width 0.2) (layer "F.Cu") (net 8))
 (segment (start 38.9 47.7) (end 38.9 49.014214) (width 0.2) (layer "F.Cu") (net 8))
 (segment (start 29 29.5) (end 29.214466 29.285534) (width 0.2) (layer "F.Cu") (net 8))
 (segment (start 34.959262 62.040738) (end 33.46967 62.040738) (width 0.2) (layer "F.Cu") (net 8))
 (segment (start 28 29.5) (end 29 29.5) (width 0.2) (layer "F.Cu") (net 8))
 (segment (start 37.5 50) (end 37.5 59.5) (width 0.2) (layer "F.Cu") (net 8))
 (segment (start 39.1 47.5) (end 38.9 47.7) (width 0.2) (layer "F.Cu") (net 8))
 (segment (start 38.9 49.014214) (end 37.914214 50) (width 0.2) (layer "F.Cu") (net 8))
 (segment (start 33.46967 62.040738) (end 32.992373 61.563441) (width 0.2) (layer "F.Cu") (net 8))
 (segment (start 29.214466 29.285534) (end 29.214466 27.95) (width 0.2) (layer "F.Cu") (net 8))
 (via (at 39.1 47.5) (size 0.6) (drill 0.3) (layers "F.Cu" "B.Cu") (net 8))
 (via (at 28 29.5) (size 0.6) (drill 0.3) (layers "F.Cu" "B.Cu") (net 8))
 (segment (start 35.5 30.5) (end 29 30.5) (width 0.2) (layer "B.Cu") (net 8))
 (segment (start 39 47.4) (end 39 34) (width 0.2) (layer "B.Cu") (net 8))
 (segment (start 39.1 47.5) (end 39 47.4) (width 0.2) (layer "B.Cu") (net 8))
 (segment (start 29 30.5) (end 28 29.5) (width 0.2) (layer "B.Cu") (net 8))
 (segment (start 39 34) (end 35.5 30.5) (width 0.2) (layer "B.Cu") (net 8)))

